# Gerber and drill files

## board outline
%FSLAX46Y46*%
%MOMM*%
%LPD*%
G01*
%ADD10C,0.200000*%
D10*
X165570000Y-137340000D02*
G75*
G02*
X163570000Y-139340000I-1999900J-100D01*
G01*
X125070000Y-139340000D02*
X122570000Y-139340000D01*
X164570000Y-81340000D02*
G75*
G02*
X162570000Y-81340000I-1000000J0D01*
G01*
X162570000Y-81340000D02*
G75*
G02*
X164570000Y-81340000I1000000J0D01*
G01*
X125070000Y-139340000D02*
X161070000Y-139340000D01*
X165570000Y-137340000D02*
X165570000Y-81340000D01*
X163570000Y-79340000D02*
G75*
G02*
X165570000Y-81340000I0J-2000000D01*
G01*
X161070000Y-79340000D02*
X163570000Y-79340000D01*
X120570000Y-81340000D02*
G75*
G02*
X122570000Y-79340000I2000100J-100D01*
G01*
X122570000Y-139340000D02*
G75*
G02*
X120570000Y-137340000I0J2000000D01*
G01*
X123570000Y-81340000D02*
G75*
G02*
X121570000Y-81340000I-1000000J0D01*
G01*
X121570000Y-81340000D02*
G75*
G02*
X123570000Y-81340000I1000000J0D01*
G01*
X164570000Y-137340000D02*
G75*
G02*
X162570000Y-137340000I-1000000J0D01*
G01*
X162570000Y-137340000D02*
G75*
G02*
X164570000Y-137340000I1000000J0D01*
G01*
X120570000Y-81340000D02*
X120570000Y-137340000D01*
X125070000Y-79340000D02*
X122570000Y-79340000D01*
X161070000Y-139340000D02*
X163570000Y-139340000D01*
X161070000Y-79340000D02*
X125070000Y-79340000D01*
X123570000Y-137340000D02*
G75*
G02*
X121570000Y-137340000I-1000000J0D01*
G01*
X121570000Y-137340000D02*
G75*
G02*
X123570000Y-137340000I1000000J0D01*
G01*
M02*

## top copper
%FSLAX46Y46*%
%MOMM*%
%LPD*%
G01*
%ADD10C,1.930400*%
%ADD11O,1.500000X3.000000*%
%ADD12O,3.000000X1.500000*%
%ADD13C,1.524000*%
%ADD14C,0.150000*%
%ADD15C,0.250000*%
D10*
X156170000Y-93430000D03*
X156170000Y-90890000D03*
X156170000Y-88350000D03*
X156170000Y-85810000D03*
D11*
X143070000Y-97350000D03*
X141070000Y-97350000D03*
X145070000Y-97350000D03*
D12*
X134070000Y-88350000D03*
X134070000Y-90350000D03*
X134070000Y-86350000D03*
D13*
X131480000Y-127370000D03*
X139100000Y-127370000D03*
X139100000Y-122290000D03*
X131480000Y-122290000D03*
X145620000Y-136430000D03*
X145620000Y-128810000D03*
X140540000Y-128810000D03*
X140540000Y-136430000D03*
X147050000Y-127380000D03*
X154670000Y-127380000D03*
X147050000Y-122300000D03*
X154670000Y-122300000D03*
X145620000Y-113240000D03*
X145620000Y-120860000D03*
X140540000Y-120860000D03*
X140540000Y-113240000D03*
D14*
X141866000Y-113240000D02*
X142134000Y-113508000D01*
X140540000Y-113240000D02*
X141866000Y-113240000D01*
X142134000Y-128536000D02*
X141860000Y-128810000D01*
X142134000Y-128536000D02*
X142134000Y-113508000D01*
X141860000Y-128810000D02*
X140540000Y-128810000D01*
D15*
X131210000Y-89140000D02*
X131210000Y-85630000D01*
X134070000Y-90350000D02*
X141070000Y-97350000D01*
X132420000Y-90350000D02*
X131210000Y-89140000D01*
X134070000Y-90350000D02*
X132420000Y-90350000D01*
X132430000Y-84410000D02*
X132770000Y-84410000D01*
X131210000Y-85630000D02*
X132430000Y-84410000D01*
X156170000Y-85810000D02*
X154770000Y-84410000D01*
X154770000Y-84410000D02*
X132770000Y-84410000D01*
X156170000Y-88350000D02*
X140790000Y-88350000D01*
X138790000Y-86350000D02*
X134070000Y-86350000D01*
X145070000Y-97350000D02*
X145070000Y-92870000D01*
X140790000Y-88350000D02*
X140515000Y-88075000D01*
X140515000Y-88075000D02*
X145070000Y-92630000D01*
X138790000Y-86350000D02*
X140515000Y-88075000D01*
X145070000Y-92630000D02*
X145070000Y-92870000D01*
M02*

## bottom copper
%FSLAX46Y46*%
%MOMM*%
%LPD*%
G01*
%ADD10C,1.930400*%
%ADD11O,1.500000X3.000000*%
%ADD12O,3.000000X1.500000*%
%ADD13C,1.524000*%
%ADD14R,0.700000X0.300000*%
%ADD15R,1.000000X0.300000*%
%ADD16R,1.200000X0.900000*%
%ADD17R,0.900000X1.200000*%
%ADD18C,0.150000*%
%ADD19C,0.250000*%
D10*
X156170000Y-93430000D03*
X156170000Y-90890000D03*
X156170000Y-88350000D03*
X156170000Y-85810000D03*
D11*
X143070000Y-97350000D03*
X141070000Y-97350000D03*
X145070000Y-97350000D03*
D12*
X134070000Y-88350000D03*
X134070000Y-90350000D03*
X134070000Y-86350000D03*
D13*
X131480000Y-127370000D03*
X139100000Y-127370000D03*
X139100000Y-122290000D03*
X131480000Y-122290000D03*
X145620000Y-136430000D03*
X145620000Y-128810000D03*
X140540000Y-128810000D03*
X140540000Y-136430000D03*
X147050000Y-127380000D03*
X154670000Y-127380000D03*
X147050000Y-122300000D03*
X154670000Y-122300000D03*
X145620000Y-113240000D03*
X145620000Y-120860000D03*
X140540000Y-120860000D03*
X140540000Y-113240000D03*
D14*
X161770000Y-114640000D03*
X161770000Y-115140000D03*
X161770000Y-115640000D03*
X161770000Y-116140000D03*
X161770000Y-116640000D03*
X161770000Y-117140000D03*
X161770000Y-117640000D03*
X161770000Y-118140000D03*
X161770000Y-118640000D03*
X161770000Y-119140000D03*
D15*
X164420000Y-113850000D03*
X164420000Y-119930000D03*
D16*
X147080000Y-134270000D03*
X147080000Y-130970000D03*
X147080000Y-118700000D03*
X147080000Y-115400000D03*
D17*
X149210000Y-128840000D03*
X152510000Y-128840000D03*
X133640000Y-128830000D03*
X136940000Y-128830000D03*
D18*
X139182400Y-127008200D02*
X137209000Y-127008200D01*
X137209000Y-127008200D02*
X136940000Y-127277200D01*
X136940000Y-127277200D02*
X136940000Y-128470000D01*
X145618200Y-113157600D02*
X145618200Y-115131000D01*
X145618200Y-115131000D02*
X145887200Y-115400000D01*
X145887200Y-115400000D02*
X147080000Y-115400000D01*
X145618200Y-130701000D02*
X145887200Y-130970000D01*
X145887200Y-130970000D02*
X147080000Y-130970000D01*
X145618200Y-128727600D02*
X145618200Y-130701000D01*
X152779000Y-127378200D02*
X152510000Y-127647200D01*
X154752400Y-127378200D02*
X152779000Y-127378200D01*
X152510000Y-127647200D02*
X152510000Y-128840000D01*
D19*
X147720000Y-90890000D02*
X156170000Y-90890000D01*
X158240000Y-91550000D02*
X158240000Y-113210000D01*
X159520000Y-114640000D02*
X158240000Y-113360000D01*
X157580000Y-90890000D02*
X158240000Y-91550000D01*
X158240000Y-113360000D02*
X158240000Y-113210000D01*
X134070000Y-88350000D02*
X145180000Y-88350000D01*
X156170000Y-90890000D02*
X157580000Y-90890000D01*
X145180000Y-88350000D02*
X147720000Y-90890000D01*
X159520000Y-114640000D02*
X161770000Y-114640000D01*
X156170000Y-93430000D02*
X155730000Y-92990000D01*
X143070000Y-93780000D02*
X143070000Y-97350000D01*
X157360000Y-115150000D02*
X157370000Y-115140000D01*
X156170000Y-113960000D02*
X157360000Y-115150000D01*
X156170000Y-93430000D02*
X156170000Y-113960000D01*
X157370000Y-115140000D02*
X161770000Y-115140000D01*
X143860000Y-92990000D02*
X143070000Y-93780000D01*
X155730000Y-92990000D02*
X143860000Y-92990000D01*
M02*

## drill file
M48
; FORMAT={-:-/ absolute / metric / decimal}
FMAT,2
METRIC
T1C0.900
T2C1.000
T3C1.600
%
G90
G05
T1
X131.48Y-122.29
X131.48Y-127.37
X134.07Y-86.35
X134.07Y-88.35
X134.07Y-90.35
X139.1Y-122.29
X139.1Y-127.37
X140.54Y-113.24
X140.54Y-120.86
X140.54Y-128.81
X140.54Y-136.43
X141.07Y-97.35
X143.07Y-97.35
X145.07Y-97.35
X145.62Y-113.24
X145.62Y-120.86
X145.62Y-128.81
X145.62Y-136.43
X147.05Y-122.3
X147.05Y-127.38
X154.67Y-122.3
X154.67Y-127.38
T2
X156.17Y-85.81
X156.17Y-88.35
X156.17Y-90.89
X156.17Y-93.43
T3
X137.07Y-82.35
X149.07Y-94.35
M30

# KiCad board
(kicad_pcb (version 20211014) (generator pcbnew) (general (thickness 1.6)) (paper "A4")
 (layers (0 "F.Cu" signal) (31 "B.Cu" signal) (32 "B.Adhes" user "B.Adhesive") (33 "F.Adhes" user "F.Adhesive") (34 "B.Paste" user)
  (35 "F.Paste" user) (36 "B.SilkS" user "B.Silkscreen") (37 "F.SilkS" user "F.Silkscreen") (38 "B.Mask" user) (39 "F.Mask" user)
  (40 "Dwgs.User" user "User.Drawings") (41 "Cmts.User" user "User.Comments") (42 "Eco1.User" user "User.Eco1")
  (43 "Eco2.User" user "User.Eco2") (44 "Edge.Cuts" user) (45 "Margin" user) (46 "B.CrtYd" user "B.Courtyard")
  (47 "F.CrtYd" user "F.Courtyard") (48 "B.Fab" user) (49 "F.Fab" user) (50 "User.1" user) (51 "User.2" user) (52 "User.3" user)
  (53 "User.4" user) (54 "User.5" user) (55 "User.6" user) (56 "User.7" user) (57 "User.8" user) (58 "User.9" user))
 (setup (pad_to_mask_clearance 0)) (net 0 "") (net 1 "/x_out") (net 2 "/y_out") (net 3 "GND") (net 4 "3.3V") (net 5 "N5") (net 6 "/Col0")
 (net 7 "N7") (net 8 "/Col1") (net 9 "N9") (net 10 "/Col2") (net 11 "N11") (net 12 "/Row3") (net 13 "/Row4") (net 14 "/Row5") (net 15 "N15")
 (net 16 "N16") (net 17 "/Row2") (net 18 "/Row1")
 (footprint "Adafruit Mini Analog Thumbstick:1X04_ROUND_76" (layer "F.Cu") (at 156.17 89.62 90)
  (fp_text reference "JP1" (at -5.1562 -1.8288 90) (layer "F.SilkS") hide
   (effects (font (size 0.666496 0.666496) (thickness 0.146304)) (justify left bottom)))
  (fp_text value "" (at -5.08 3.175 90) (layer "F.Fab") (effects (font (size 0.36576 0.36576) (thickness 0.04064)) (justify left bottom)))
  (pad "1" thru_hole circle (at -3.81 0 180) (size 1.9304 1.9304) (drill 1) (layers *.Cu *.Mask) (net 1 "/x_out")
   (solder_mask_margin 0.0508))
  (pad "2" thru_hole circle (at -1.27 0 180) (size 1.9304 1.9304) (drill 1) (layers *.Cu *.Mask) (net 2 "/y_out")
   (solder_mask_margin 0.0508))
  (pad "3" thru_hole circle (at 1.27 0 180) (size 1.9304 1.9304) (drill 1) (layers *.Cu *.Mask) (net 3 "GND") (solder_mask_margin 0.0508))
  (pad "4" thru_hole circle (at 3.81 0 180) (size 1.9304 1.9304) (drill 1) (layers *.Cu *.Mask) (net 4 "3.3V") (solder_mask_margin 0.0508)))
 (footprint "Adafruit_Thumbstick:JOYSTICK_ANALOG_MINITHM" (layer "F.Cu") (at 143.07 88.35 180)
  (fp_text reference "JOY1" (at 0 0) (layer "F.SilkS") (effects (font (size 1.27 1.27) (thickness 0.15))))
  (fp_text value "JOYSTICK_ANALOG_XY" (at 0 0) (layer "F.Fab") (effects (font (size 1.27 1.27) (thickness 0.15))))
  (pad "" np_thru_hole circle (at -6 -6 180) (size 1.6 1.6) (drill 1.6) (layers *.Cu *.Mask))
  (pad "" np_thru_hole circle (at 6 6 180) (size 1.6 1.6) (drill 1.6) (layers *.Cu *.Mask))
  (pad "X" thru_hole oval (at 0 -9 270) (size 3 1.5) (drill 0.9) (layers *.Cu *.Mask) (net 1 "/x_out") (solder_mask_margin 0.0508))
  (pad "X+" thru_hole oval (at 2 -9 270) (size 3 1.5) (drill 0.9) (layers *.Cu *.Mask) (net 4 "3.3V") (solder_mask_margin 0.0508))
  (pad "X-" thru_hole oval (at -2 -9 270) (size 3 1.5) (drill 0.9) (layers *.Cu *.Mask) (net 3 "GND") (solder_mask_margin 0.0508))
  (pad "Y" thru_hole oval (at 9 0 180) (size 3 1.5) (drill 0.9) (layers *.Cu *.Mask) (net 2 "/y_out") (solder_mask_margin 0.0508))
  (pad "Y+" thru_hole oval (at 9 -2 180) (size 3 1.5) (drill 0.9) (layers *.Cu *.Mask) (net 4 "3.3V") (solder_mask_margin 0.0508))
  (pad "Y-" thru_hole oval (at 9 2 180) (size 3 1.5) (drill 0.9) (layers *.Cu *.Mask) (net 3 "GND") (solder_mask_margin 0.0508)))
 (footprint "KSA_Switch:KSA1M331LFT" (layer "F.Cu") (at 135.29 124.83 90)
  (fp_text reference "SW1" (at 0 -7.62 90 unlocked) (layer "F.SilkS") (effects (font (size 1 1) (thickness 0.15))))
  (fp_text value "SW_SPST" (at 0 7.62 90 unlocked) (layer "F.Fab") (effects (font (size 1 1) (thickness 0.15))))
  (pad "1" thru_hole circle (at -2.54 -3.81 90) (size 1.524 1.524) (drill 0.9) (layers *.Cu *.Mask) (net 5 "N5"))
  (pad "1" thru_hole circle (at -2.54 3.81 90) (size 1.524 1.524) (drill 0.9) (layers *.Cu *.Mask) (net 5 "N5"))
  (pad "2" thru_hole circle (at 2.54 3.81 90) (size 1.524 1.524) (drill 0.9) (layers *.Cu *.Mask) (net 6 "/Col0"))
  (pad "2" thru_hole circle (at 2.54 -3.81 90) (size 1.524 1.524) (drill 0.9) (layers *.Cu *.Mask) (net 6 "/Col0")))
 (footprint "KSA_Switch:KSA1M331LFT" (layer "F.Cu") (at 143.08 132.62 180)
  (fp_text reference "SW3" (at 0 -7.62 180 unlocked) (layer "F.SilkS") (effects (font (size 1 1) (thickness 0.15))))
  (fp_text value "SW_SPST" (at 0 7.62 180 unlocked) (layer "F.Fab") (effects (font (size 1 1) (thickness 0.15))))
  (pad "1" thru_hole circle (at -2.54 -3.81 180) (size 1.524 1.524) (drill 0.9) (layers *.Cu *.Mask) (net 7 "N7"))
  (pad "1" thru_hole circle (at -2.54 3.81 180) (size 1.524 1.524) (drill 0.9) (layers *.Cu *.Mask) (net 7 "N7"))
  (pad "2" thru_hole circle (at 2.54 3.81 180) (size 1.524 1.524) (drill 0.9) (layers *.Cu *.Mask) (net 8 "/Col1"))
  (pad "2" thru_hole circle (at 2.54 -3.81 180) (size 1.524 1.524) (drill 0.9) (layers *.Cu *.Mask) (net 8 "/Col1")))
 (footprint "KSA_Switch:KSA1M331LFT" (layer "F.Cu") (at 150.86 124.84 90)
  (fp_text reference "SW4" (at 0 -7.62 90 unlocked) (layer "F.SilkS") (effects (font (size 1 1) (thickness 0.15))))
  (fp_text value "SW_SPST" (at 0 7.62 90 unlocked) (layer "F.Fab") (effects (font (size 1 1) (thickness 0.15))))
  (pad "1" thru_hole circle (at -2.54 -3.81 90) (size 1.524 1.524) (drill 0.9) (layers *.Cu *.Mask) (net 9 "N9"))
  (pad "1" thru_hole circle (at -2.54 3.81 90) (size 1.524 1.524) (drill 0.9) (layers *.Cu *.Mask) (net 9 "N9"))
  (pad "2" thru_hole circle (at 2.54 -3.81 90) (size 1.524 1.524) (drill 0.9) (layers *.Cu *.Mask) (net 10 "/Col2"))
  (pad "2" thru_hole circle (at 2.54 3.81 90) (size 1.524 1.524) (drill 0.9) (layers *.Cu *.Mask) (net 10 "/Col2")))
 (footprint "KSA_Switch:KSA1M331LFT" (layer "F.Cu") (at 143.08 117.05 180)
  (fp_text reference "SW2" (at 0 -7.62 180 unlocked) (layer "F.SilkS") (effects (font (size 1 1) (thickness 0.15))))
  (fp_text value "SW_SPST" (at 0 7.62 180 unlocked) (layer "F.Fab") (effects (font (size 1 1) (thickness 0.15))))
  (pad "1" thru_hole circle (at -2.54 3.81 180) (size 1.524 1.524) (drill 0.9) (layers *.Cu *.Mask) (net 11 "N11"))
  (pad "1" thru_hole circle (at -2.54 -3.81 180) (size 1.524 1.524) (drill 0.9) (layers *.Cu *.Mask) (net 11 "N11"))
  (pad "2" thru_hole circle (at 2.54 -3.81 180) (size 1.524 1.524) (drill 0.9) (layers *.Cu *.Mask) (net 8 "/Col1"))
  (pad "2" thru_hole circle (at 2.54 3.81 180) (size 1.524 1.524) (drill 0.9) (layers *.Cu *.Mask) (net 8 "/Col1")))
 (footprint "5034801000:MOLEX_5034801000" (layer "B.Cu") (at 161.77 116.89 -90)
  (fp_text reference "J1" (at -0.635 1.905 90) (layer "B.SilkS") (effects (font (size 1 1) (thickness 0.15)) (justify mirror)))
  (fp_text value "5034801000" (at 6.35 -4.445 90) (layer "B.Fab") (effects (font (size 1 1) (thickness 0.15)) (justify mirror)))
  (pad "1" smd rect locked (at -2.25 0 270) (size 0.3 0.7) (layers "B.Cu" "B.Paste" "B.Mask") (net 2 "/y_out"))
  (pad "2" smd rect locked (at -1.75 0 270) (size 0.3 0.7) (layers "B.Cu" "B.Paste" "B.Mask") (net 1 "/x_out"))
  (pad "3" smd rect locked (at -1.25 0 270) (size 0.3 0.7) (layers "B.Cu" "B.Paste" "B.Mask") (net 10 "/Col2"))
  (pad "4" smd rect locked (at -0.75 0 270) (size 0.3 0.7) (layers "B.Cu" "B.Paste" "B.Mask") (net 8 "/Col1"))
  (pad "5" smd rect locked (at -0.25 0 270) (size 0.3 0.7) (layers "B.Cu" "B.Paste" "B.Mask") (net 6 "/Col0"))
  (pad "6" smd rect locked (at 0.25 0 270) (size 0.3 0.7) (layers "B.Cu" "B.Paste" "B.Mask") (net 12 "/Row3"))
  (pad "7" smd rect locked (at 0.75 0 270) (size 0.3 0.7) (layers "B.Cu" "B.Paste" "B.Mask") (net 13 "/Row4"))
  (pad "8" smd rect locked (at 1.25 0 270) (size 0.3 0.7) (layers "B.Cu" "B.Paste" "B.Mask") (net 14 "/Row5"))
  (pad "9" smd rect locked (at 1.75 0 270) (size 0.3 0.7) (layers "B.Cu" "B.Paste" "B.Mask") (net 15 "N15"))
  (pad "10" smd rect locked (at 2.25 0 270) (size 0.3 0.7) (layers "B.Cu" "B.Paste" "B.Mask") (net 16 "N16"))
  (pad "S1" smd rect locked (at -3.04 -2.65 270) (size 0.3 1) (layers "B.Cu" "B.Paste" "B.Mask") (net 3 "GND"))
  (pad "S2" smd rect locked (at 3.04 -2.65 270) (size 0.3 1) (layers "B.Cu" "B.Paste" "B.Mask") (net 3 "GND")))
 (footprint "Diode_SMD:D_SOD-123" (layer "B.Cu") (at 147.08 132.62 90)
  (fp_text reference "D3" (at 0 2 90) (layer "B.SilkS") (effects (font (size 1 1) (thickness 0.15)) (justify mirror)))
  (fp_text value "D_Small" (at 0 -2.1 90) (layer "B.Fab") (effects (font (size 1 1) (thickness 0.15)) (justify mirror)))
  (pad "1" smd rect (at -1.65 0 90) (size 0.9 1.2) (layers "B.Cu" "B.Paste" "B.Mask") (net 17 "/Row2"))
  (pad "2" smd rect (at 1.65 0 90) (size 0.9 1.2) (layers "B.Cu" "B.Paste" "B.Mask") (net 7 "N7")))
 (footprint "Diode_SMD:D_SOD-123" (layer "B.Cu") (at 147.08 117.05 90)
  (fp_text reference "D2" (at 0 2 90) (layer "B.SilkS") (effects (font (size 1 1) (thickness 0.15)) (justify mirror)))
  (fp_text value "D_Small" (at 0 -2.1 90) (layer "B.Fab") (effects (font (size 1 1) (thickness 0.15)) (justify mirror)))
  (pad "1" smd rect (at -1.65 0 90) (size 0.9 1.2) (layers "B.Cu" "B.Paste" "B.Mask") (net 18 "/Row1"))
  (pad "2" smd rect (at 1.65 0 90) (size 0.9 1.2) (layers "B.Cu" "B.Paste" "B.Mask") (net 11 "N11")))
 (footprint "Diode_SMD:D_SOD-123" (layer "B.Cu") (at 150.86 128.84)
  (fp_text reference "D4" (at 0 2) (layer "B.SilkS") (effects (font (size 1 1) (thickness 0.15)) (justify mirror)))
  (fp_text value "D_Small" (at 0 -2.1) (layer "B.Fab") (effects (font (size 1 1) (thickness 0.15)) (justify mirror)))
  (pad "1" smd rect (at -1.65 0) (size 0.9 1.2) (layers "B.Cu" "B.Paste" "B.Mask") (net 17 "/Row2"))
  (pad "2" smd rect (at 1.65 0) (size 0.9 1.2) (layers "B.Cu" "B.Paste" "B.Mask") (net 9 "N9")))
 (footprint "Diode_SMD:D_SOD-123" (layer "B.Cu") (at 135.29 128.83)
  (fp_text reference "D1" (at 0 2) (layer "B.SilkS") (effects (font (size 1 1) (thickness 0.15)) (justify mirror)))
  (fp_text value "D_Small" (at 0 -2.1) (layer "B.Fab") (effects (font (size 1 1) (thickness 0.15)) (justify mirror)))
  (pad "1" smd rect (at -1.65 0) (size 0.9 1.2) (layers "B.Cu" "B.Paste" "B.Mask") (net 17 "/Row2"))
  (pad "2" smd rect (at 1.65 0) (size 0.9 1.2) (layers "B.Cu" "B.Paste" "B.Mask") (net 5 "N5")))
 (gr_arc (start 165.57 137.34) (mid 164.984227 138.754245) (end 163.57 139.34) (layer "Edge.Cuts") (width 0.2))
 (gr_line (start 125.07 139.34) (end 122.57 139.34) (layer "Edge.Cuts") (width 0.2))
 (gr_circle (center 163.57 81.34) (end 164.57 81.34) (layer "Edge.Cuts") (width 0.2) (fill none))
 (gr_line (start 125.07 139.34) (end 161.07 139.34) (layer "Edge.Cuts") (width 0.2))
 (gr_line (start 165.57 137.34) (end 165.57 81.34) (layer "Edge.Cuts") (width 0.2))
 (gr_arc (start 163.57 79.34) (mid 164.98421 79.925793) (end 165.57 81.34) (layer "Edge.Cuts") (width 0.2))
 (gr_line (start 161.07 79.34) (end 163.57 79.34) (layer "Edge.Cuts") (width 0.2))
 (gr_arc (start 120.57 81.34) (mid 121.1558 79.925818) (end 122.57 79.34) (layer "Edge.Cuts") (width 0.2))
 (gr_arc (start 122.57 139.34) (mid 121.155783 138.75422) (end 120.57 137.34) (layer "Edge.Cuts") (width 0.2))
 (gr_circle (center 122.57 81.34) (end 123.57 81.34) (layer "Edge.Cuts") (width 0.2) (fill none))
 (gr_circle (center 163.57 137.34) (end 164.57 137.34) (layer "Edge.Cuts") (width 0.2) (fill none))
 (gr_line (start 120.57 81.34) (end 120.57 137.34) (layer "Edge.Cuts") (width 0.2))
 (gr_line (start 125.07 79.34) (end 122.57 79.34) (layer "Edge.Cuts") (width 0.2))
 (gr_line (start 161.07 139.34) (end 163.57 139.34) (layer "Edge.Cuts") (width 0.2))
 (gr_line (start 161.07 79.34) (end 125.07 79.34) (layer "Edge.Cuts") (width 0.2))
 (gr_circle (center 122.57 137.34) (end 123.57 137.34) (layer "Edge.Cuts") (width 0.2) (fill none))
 (segment (start 139.1824 127.0082) (end 137.209 127.0082) (width 0.15) (layer "B.Cu") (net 5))
 (segment (start 137.209 127.0082) (end 136.94 127.2772) (width 0.15) (layer "B.Cu") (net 5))
 (segment (start 136.94 127.2772) (end 136.94 128.47) (width 0.15) (layer "B.Cu") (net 5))
 (segment (start 145.6182 113.1576) (end 145.6182 115.131) (width 0.15) (layer "B.Cu") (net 11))
 (segment (start 145.6182 115.131) (end 145.8872 115.4) (width 0.15) (layer "B.Cu") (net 11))
 (segment (start 145.8872 115.4) (end 147.08 115.4) (width 0.15) (layer "B.Cu") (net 11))
 (segment (start 145.6182 130.701) (end 145.8872 130.97) (width 0.15) (layer "B.Cu") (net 7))
 (segment (start 145.8872 130.97) (end 147.08 130.97) (width 0.15) (layer "B.Cu") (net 7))
 (segment (start 145.6182 128.7276) (end 145.6182 130.701) (width 0.15) (layer "B.Cu") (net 7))
 (segment (start 152.779 127.3782) (end 152.51 127.6472) (width 0.15) (layer "B.Cu") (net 9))
 (segment (start 154.7524 127.3782) (end 152.779 127.3782) (width 0.15) (layer "B.Cu") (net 9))
 (segment (start 152.51 127.6472) (end 152.51 128.84) (width 0.15) (layer "B.Cu") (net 9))
 (segment (start 141.866 113.24) (end 142.134 113.508) (width 0.15) (layer "F.Cu") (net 8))
 (segment (start 140.54 113.24) (end 141.866 113.24) (width 0.15) (layer "F.Cu") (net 8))
 (segment (start 142.134 128.536) (end 141.86 128.81) (width 0.15) (layer "F.Cu") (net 8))
 (segment (start 142.134 128.536) (end 142.134 113.508) (width 0.15) (layer "F.Cu") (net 8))
 (segment (start 141.86 128.81) (end 140.54 128.81) (width 0.15) (layer "F.Cu") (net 8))
 (segment (start 131.21 89.14) (end 131.21 85.63) (width 0.25) (layer "F.Cu") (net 4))
 (segment (start 134.07 90.35) (end 141.07 97.35) (width 0.25) (layer "F.Cu") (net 4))
 (segment (start 132.42 90.35) (end 131.21 89.14) (width 0.25) (layer "F.Cu") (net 4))
 (segment (start 134.07 90.35) (end 132.42 90.35) (width 0.25) (layer "F.Cu") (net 4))
 (segment (start 132.43 84.41) (end 132.77 84.41) (width 0.25) (layer "F.Cu") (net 4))
 (segment (start 131.21 85.63) (end 132.43 84.41) (width 0.25) (layer "F.Cu") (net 4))
 (segment (start 156.17 85.81) (end 154.77 84.41) (width 0.25) (layer "F.Cu") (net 4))
 (segment (start 154.77 84.41) (end 132.77 84.41) (width 0.25) (layer "F.Cu") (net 4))
 (segment (start 156.17 88.35) (end 140.79 88.35) (width 0.25) (layer "F.Cu") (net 3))
 (segment (start 138.79 86.35) (end 134.07 86.35) (width 0.25) (layer "F.Cu") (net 3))
 (segment (start 145.07 97.35) (end 145.07 92.87) (width 0.25) (layer "F.Cu") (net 3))
 (segment (start 140.79 88.35) (end 140.515 88.075) (width 0.25) (layer "F.Cu") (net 3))
 (segment (start 140.515 88.075) (end 145.07 92.63) (width 0.25) (layer "F.Cu") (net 3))
 (segment (start 138.79 86.35) (end 140.515 88.075) (width 0.25) (layer "F.Cu") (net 3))
 (segment (start 145.07 92.63) (end 145.07 92.87) (width 0.25) (layer "F.Cu") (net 3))
 (segment (start 147.72 90.89) (end 156.17 90.89) (width 0.25) (layer "B.Cu") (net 2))
 (segment (start 158.24 91.55) (end 158.24 113.21) (width 0.25) (layer "B.Cu") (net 2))
 (segment (start 159.52 114.64) (end 158.24 113.36) (width 0.25) (layer "B.Cu") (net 2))
 (segment (start 157.58 90.89) (end 158.24 91.55) (width 0.25) (layer "B.Cu") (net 2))
 (segment (start 158.24 113.36) (end 158.24 113.21) (width 0.25) (layer "B.Cu") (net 2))
 (segment (start 134.07 88.35) (end 145.18 88.35) (width 0.25) (layer "B.Cu") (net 2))
 (segment (start 156.17 90.89) (end 157.58 90.89) (width 0.25) (layer "B.Cu") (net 2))
 (segment (start 145.18 88.35) (end 147.72 90.89) (width 0.25) (layer "B.Cu") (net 2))
 (segment (start 159.52 114.64) (end 161.77 114.64) (width 0.25) (layer "B.Cu") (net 2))
 (segment (start 156.17 93.43) (end 155.73 92.99) (width 0.25) (layer "B.Cu") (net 1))
 (segment (start 143.07 93.78) (end 143.07 97.35) (width 0.25) (layer "B.Cu") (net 1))
 (segment (start 157.36 115.15) (end 157.37 115.14) (width 0.25) (layer "B.Cu") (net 1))
 (segment (start 156.17 113.96) (end 157.36 115.15) (width 0.25) (layer "B.Cu") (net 1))
 (segment (start 156.17 93.43) (end 156.17 113.96) (width 0.25) (layer "B.Cu") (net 1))
 (segment (start 157.37 115.14) (end 161.77 115.14) (width 0.25) (layer "B.Cu") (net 1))
 (segment (start 143.86 92.99) (end 143.07 93.78) (width 0.25) (layer "B.Cu") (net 1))
 (segment (start 155.73 92.99) (end 143.86 92.99) (width 0.25) (layer "B.Cu") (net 1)))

